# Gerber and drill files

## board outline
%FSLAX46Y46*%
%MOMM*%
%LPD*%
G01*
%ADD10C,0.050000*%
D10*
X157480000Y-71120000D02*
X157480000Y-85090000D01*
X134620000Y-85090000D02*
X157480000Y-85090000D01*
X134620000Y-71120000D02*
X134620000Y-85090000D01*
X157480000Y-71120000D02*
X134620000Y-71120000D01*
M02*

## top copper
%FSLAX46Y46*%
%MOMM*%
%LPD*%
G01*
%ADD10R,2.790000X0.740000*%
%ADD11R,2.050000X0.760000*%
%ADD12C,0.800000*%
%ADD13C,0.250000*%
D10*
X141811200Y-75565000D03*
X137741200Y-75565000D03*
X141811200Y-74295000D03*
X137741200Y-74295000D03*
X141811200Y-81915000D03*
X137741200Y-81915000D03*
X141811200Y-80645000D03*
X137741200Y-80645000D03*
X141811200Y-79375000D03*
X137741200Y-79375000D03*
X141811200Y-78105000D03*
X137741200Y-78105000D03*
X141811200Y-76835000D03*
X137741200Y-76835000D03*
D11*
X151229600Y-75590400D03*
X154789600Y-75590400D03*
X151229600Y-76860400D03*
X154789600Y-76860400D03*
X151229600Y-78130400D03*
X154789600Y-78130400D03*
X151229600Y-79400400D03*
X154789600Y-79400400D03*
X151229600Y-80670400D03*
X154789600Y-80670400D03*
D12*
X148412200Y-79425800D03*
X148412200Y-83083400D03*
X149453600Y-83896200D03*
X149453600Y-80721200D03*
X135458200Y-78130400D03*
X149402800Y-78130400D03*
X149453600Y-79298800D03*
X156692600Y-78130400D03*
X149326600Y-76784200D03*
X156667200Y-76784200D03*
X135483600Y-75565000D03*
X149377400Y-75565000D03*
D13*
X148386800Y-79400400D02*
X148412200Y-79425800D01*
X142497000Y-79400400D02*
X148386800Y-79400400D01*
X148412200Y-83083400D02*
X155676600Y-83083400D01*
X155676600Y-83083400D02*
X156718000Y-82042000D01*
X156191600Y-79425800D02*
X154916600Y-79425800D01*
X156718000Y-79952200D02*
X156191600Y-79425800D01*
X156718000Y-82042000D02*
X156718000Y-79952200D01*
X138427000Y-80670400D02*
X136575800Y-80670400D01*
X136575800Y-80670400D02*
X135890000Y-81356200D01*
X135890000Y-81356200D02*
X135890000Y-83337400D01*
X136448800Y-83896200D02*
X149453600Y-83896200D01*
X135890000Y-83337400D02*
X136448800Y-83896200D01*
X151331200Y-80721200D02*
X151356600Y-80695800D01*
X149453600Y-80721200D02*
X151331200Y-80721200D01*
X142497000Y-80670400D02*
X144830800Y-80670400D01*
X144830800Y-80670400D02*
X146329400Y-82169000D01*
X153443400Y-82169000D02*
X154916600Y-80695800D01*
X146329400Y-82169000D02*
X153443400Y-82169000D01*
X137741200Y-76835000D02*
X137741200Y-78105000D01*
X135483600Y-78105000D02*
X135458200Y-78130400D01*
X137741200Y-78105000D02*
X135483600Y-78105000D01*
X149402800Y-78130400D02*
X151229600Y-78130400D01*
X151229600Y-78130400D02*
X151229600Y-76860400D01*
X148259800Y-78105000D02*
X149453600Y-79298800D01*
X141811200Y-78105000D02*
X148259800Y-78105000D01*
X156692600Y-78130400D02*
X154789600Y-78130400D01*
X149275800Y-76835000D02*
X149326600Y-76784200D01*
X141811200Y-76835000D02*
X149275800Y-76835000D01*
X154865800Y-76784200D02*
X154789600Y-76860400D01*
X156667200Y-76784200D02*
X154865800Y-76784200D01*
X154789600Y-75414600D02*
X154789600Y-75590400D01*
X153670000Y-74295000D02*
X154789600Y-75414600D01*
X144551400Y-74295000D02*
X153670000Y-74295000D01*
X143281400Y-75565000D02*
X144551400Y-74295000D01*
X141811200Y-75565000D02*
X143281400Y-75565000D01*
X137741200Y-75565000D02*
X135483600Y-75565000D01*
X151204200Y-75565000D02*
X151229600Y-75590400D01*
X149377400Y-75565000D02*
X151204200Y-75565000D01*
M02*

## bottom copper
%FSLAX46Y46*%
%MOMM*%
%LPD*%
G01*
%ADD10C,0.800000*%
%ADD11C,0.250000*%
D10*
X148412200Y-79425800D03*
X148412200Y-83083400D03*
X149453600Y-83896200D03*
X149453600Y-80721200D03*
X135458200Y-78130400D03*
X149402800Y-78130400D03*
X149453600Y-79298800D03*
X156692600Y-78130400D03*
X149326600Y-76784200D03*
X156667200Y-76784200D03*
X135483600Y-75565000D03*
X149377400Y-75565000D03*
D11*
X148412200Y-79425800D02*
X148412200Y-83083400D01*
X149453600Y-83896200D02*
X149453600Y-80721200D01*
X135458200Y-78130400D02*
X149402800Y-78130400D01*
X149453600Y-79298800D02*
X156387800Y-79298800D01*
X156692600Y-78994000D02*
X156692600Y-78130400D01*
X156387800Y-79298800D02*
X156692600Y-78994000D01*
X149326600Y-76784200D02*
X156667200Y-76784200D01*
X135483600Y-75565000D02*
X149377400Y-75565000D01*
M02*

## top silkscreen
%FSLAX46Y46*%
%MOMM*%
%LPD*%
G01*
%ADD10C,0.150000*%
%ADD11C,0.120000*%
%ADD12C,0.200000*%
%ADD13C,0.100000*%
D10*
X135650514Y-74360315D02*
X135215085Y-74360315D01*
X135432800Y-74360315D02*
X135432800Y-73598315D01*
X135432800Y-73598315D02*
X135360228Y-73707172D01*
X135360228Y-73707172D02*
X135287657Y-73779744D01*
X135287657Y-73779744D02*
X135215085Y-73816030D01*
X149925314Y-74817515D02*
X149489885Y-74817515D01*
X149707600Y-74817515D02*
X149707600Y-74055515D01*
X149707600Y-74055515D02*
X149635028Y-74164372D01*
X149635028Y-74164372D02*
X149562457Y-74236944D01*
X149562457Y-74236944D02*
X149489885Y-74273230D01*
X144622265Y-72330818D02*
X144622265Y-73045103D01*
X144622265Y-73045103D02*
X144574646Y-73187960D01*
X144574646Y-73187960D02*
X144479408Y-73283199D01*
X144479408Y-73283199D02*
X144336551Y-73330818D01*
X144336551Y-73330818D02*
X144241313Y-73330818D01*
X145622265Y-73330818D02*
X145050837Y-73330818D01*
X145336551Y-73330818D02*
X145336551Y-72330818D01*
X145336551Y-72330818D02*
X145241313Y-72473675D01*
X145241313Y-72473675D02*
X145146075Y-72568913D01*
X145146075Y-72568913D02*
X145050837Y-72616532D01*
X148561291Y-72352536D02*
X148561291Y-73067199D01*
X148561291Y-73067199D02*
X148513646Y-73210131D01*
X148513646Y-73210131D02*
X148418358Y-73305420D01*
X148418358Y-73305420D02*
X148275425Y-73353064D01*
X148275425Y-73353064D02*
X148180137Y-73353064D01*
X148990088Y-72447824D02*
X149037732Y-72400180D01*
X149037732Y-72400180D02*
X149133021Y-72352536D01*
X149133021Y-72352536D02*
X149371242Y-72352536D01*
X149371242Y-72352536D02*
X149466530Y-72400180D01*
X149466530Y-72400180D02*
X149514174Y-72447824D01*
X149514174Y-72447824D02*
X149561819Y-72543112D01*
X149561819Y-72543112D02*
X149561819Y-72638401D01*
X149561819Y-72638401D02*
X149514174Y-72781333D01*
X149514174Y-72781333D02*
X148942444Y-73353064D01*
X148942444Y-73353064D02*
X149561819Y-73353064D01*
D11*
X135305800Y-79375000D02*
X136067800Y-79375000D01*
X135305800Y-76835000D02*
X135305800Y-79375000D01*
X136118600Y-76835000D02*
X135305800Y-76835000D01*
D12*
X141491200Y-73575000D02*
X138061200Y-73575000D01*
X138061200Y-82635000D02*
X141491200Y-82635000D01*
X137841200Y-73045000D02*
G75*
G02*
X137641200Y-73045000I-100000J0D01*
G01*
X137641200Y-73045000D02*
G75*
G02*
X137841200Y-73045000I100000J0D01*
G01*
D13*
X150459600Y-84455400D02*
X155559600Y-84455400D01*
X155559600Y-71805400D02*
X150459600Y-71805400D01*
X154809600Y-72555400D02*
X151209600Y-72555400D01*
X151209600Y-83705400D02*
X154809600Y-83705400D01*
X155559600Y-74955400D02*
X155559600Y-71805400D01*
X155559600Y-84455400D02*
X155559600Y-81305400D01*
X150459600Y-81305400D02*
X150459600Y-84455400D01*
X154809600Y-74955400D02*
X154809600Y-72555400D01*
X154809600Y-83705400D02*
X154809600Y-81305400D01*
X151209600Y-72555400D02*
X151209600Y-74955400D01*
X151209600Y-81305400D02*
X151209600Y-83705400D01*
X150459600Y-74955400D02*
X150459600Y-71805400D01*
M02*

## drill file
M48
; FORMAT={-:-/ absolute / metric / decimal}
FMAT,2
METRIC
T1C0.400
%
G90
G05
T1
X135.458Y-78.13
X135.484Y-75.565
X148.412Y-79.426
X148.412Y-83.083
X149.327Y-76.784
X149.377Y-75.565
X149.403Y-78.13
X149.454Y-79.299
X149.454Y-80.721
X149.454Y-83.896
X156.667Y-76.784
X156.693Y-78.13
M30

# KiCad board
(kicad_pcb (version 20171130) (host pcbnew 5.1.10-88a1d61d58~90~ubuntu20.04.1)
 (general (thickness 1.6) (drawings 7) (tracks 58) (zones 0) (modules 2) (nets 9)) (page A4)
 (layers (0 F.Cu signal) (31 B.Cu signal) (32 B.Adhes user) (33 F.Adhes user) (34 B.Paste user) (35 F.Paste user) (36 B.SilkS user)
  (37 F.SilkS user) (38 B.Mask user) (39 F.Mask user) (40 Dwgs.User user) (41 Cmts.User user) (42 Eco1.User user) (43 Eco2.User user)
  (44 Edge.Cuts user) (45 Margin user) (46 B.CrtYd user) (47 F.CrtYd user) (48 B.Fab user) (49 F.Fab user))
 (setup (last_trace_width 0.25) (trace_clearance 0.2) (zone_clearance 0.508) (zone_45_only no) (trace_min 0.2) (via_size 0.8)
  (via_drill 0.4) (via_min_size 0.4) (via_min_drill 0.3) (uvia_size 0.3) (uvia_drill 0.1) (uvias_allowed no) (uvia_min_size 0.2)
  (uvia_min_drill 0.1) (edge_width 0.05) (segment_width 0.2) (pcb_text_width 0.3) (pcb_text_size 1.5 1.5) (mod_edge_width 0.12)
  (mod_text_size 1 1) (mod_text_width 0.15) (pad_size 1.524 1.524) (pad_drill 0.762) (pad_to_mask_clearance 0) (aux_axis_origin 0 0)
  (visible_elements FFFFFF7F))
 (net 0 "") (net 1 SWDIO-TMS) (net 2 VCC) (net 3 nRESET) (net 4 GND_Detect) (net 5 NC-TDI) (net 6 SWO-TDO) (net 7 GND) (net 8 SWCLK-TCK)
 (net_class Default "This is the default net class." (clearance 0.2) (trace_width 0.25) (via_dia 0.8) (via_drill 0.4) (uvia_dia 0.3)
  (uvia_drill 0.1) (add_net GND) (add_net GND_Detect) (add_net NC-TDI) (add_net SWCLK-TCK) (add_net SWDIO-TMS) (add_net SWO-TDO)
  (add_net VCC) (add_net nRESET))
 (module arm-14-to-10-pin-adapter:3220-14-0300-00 (layer F.Cu) (at 139.7762 78.105 270)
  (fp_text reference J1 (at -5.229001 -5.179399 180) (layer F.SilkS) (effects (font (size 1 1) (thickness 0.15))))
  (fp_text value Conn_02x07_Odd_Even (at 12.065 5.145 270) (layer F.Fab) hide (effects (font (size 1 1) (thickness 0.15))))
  (fp_line (start 1.27 4.4704) (end 1.27 3.7084) (layer F.SilkS) (width 0.12))
  (fp_line (start -1.27 4.4704) (end 1.27 4.4704) (layer F.SilkS) (width 0.12))
  (fp_line (start -1.27 3.6576) (end -1.27 4.4704) (layer F.SilkS) (width 0.12))
  (fp_line (start -4.53 -1.715) (end -4.53 1.715) (layer F.SilkS) (width 0.2))
  (fp_line (start 4.53 1.715) (end 4.53 -1.715) (layer F.SilkS) (width 0.2))
  (fp_circle (center -5.06 2.035) (end -4.96 2.035) (layer F.SilkS) (width 0.2))
  (pad 4 smd rect (at -2.54 -2.035 270) (size 0.74 2.79) (layers F.Cu F.Paste F.Mask) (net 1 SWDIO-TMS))
  (pad 3 smd rect (at -2.54 2.035 270) (size 0.74 2.79) (layers F.Cu F.Paste F.Mask) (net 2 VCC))
  (pad 2 smd rect (at -3.81 -2.035 270) (size 0.74 2.79) (layers F.Cu F.Paste F.Mask))
  (pad 1 smd rect (at -3.81 2.035 270) (size 0.74 2.79) (layers F.Cu F.Paste F.Mask))
  (pad 14 smd rect (at 3.81 -2.035 270) (size 0.74 2.79) (layers F.Cu F.Paste F.Mask))
  (pad 13 smd rect (at 3.81 2.035 270) (size 0.74 2.79) (layers F.Cu F.Paste F.Mask))
  (pad 12 smd rect (at 2.54 -2.035 270) (size 0.74 2.79) (layers F.Cu F.Paste F.Mask) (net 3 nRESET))
  (pad 11 smd rect (at 2.54 2.035 270) (size 0.74 2.79) (layers F.Cu F.Paste F.Mask) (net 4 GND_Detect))
  (pad 10 smd rect (at 1.27 -2.035 270) (size 0.74 2.79) (layers F.Cu F.Paste F.Mask) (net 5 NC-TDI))
  (pad 9 smd rect (at 1.27 2.035 270) (size 0.74 2.79) (layers F.Cu F.Paste F.Mask))
  (pad 8 smd rect (at 0 -2.035 270) (size 0.74 2.79) (layers F.Cu F.Paste F.Mask) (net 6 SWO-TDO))
  (pad 7 smd rect (at 0 2.035 270) (size 0.74 2.79) (layers F.Cu F.Paste F.Mask) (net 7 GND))
  (pad 6 smd rect (at -1.27 -2.035 270) (size 0.74 2.79) (layers F.Cu F.Paste F.Mask) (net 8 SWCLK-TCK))
  (pad 5 smd rect (at -1.27 2.035 270) (size 0.74 2.79) (layers F.Cu F.Paste F.Mask) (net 7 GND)))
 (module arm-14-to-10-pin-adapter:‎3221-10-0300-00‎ (layer F.Cu) (at 153.0096 78.1304 270)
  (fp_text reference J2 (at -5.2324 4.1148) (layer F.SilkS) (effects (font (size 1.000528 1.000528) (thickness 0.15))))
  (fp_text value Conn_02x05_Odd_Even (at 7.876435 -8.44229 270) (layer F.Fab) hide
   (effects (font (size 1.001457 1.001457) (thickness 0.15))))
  (fp_line (start 6.325 2.55) (end 6.325 -2.55) (layer F.SilkS) (width 0.1))
  (fp_line (start -6.325 -2.55) (end -6.325 2.55) (layer F.SilkS) (width 0.1))
  (fp_line (start -5.575 -1.8) (end -5.575 1.8) (layer F.SilkS) (width 0.1))
  (fp_line (start 5.575 1.8) (end 5.575 -1.8) (layer F.SilkS) (width 0.1))
  (fp_line (start -3.175 -2.55) (end -6.325 -2.55) (layer F.SilkS) (width 0.1))
  (fp_line (start 6.325 -2.55) (end 3.175 -2.55) (layer F.SilkS) (width 0.1))
  (fp_line (start 3.175 2.55) (end 6.325 2.55) (layer F.SilkS) (width 0.1))
  (fp_line (start -3.175 -1.8) (end -5.575 -1.8) (layer F.SilkS) (width 0.1))
  (fp_line (start 5.575 -1.8) (end 3.175 -1.8) (layer F.SilkS) (width 0.1))
  (fp_line (start -5.575 1.8) (end -3.175 1.8) (layer F.SilkS) (width 0.1))
  (fp_line (start 3.175 1.8) (end 5.575 1.8) (layer F.SilkS) (width 0.1))
  (fp_line (start -3.175 2.55) (end -6.325 2.55) (layer F.SilkS) (width 0.1))
  (pad 1 smd rect (at -2.54 1.78 270) (size 0.76 2.05) (layers F.Cu F.Paste F.Mask) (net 2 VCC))
  (pad 2 smd rect (at -2.54 -1.78 270) (size 0.76 2.05) (layers F.Cu F.Paste F.Mask) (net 1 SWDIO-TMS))
  (pad 3 smd rect (at -1.27 1.78 270) (size 0.76 2.05) (layers F.Cu F.Paste F.Mask) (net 7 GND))
  (pad 4 smd rect (at -1.27 -1.78 270) (size 0.76 2.05) (layers F.Cu F.Paste F.Mask) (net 8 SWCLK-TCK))
  (pad 5 smd rect (at 0 1.78 270) (size 0.76 2.05) (layers F.Cu F.Paste F.Mask) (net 7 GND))
  (pad 6 smd rect (at 0 -1.78 270) (size 0.76 2.05) (layers F.Cu F.Paste F.Mask) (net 6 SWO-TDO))
  (pad 7 smd rect (at 1.27 1.78 270) (size 0.76 2.05) (layers F.Cu F.Paste F.Mask))
  (pad 8 smd rect (at 1.27 -1.78 270) (size 0.76 2.05) (layers F.Cu F.Paste F.Mask) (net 5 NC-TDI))
  (pad 9 smd rect (at 2.54 1.78 270) (size 0.76 2.05) (layers F.Cu F.Paste F.Mask) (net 4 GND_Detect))
  (pad 10 smd rect (at 2.54 -1.78 270) (size 0.76 2.05) (layers F.Cu F.Paste F.Mask) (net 3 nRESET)))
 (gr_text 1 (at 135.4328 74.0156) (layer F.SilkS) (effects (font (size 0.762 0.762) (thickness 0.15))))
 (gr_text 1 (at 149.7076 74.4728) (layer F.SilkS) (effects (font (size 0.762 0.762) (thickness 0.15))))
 (gr_line (start 157.48 71.12) (end 157.48 85.09) (layer Edge.Cuts) (width 0.05))
 (gr_line (start 134.62 85.09) (end 157.48 85.09) (layer Edge.Cuts) (width 0.05))
 (gr_line (start 134.62 71.12) (end 134.62 85.09) (layer Edge.Cuts) (width 0.05))
 (gr_line (start 157.48 71.12) (end 134.62 71.12) (layer Edge.Cuts) (width 0.05))
 (via (at 148.4122 79.4258) (size 0.8) (drill 0.4) (layers F.Cu B.Cu) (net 5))
 (segment (start 148.3868 79.4004) (end 148.4122 79.4258) (width 0.25) (layer F.Cu) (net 5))
 (segment (start 142.497 79.4004) (end 148.3868 79.4004) (width 0.25) (layer F.Cu) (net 5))
 (via (at 148.4122 83.0834) (size 0.8) (drill 0.4) (layers F.Cu B.Cu) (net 5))
 (segment (start 148.4122 79.4258) (end 148.4122 83.0834) (width 0.25) (layer B.Cu) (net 5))
 (segment (start 148.4122 83.0834) (end 155.6766 83.0834) (width 0.25) (layer F.Cu) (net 5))
 (segment (start 155.6766 83.0834) (end 156.718 82.042) (width 0.25) (layer F.Cu) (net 5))
 (segment (start 156.1916 79.4258) (end 154.9166 79.4258) (width 0.25) (layer F.Cu) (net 5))
 (segment (start 156.718 79.9522) (end 156.1916 79.4258) (width 0.25) (layer F.Cu) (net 5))
 (segment (start 156.718 82.042) (end 156.718 79.9522) (width 0.25) (layer F.Cu) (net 5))
 (segment (start 138.427 80.6704) (end 136.5758 80.6704) (width 0.25) (layer F.Cu) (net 4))
 (segment (start 136.5758 80.6704) (end 135.89 81.3562) (width 0.25) (layer F.Cu) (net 4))
 (segment (start 135.89 81.3562) (end 135.89 83.3374) (width 0.25) (layer F.Cu) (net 4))
 (via (at 149.4536 83.8962) (size 0.8) (drill 0.4) (layers F.Cu B.Cu) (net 4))
 (segment (start 136.4488 83.8962) (end 149.4536 83.8962) (width 0.25) (layer F.Cu) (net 4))
 (segment (start 135.89 83.3374) (end 136.4488 83.8962) (width 0.25) (layer F.Cu) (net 4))
 (via (at 149.4536 80.7212) (size 0.8) (drill 0.4) (layers F.Cu B.Cu) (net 4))
 (segment (start 149.4536 83.8962) (end 149.4536 80.7212) (width 0.25) (layer B.Cu) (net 4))
 (segment (start 151.3312 80.7212) (end 151.3566 80.6958) (width 0.25) (layer F.Cu) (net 4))
 (segment (start 149.4536 80.7212) (end 151.3312 80.7212) (width 0.25) (layer F.Cu) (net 4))
 (segment (start 142.497 80.6704) (end 144.8308 80.6704) (width 0.25) (layer F.Cu) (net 3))
 (segment (start 144.8308 80.6704) (end 146.3294 82.169) (width 0.25) (layer F.Cu) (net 3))
 (segment (start 153.4434 82.169) (end 154.9166 80.6958) (width 0.25) (layer F.Cu) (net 3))
 (segment (start 146.3294 82.169) (end 153.4434 82.169) (width 0.25) (layer F.Cu) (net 3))
 (segment (start 137.7412 76.835) (end 137.7412 78.105) (width 0.25) (layer F.Cu) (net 7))
 (segment (start 135.4836 78.105) (end 135.4582 78.1304) (width 0.25) (layer F.Cu) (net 7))
 (via (at 135.4582 78.1304) (size 0.8) (drill 0.4) (layers F.Cu B.Cu) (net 7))
 (segment (start 137.7412 78.105) (end 135.4836 78.105) (width 0.25) (layer F.Cu) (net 7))
 (via (at 149.4028 78.1304) (size 0.8) (drill 0.4) (layers F.Cu B.Cu) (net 7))
 (segment (start 135.4582 78.1304) (end 149.4028 78.1304) (width 0.25) (layer B.Cu) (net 7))
 (segment (start 149.4028 78.1304) (end 151.2296 78.1304) (width 0.25) (layer F.Cu) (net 7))
 (segment (start 151.2296 78.1304) (end 151.2296 76.8604) (width 0.25) (layer F.Cu) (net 7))
 (via (at 149.4536 79.2988) (size 0.8) (drill 0.4) (layers F.Cu B.Cu) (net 6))
 (segment (start 148.2598 78.105) (end 149.4536 79.2988) (width 0.25) (layer F.Cu) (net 6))
 (segment (start 141.8112 78.105) (end 148.2598 78.105) (width 0.25) (layer F.Cu) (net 6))
 (segment (start 149.4536 79.2988) (end 156.3878 79.2988) (width 0.25) (layer B.Cu) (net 6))
 (via (at 156.6926 78.1304) (size 0.8) (drill 0.4) (layers F.Cu B.Cu) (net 6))
 (segment (start 156.6926 78.994) (end 156.6926 78.1304) (width 0.25) (layer B.Cu) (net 6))
 (segment (start 156.3878 79.2988) (end 156.6926 78.994) (width 0.25) (layer B.Cu) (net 6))
 (segment (start 156.6926 78.1304) (end 154.7896 78.1304) (width 0.25) (layer F.Cu) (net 6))
 (via (at 149.3266 76.7842) (size 0.8) (drill 0.4) (layers F.Cu B.Cu) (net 8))
 (segment (start 149.2758 76.835) (end 149.3266 76.7842) (width 0.25) (layer F.Cu) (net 8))
 (segment (start 141.8112 76.835) (end 149.2758 76.835) (width 0.25) (layer F.Cu) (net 8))
 (via (at 156.6672 76.7842) (size 0.8) (drill 0.4) (layers F.Cu B.Cu) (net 8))
 (segment (start 149.3266 76.7842) (end 156.6672 76.7842) (width 0.25) (layer B.Cu) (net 8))
 (segment (start 154.8658 76.7842) (end 154.7896 76.8604) (width 0.25) (layer F.Cu) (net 8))
 (segment (start 156.6672 76.7842) (end 154.8658 76.7842) (width 0.25) (layer F.Cu) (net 8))
 (segment (start 154.7896 75.4146) (end 154.7896 75.5904) (width 0.25) (layer F.Cu) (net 1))
 (segment (start 153.67 74.295) (end 154.7896 75.4146) (width 0.25) (layer F.Cu) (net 1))
 (segment (start 144.5514 74.295) (end 153.67 74.295) (width 0.25) (layer F.Cu) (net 1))
 (segment (start 143.2814 75.565) (end 144.5514 74.295) (width 0.25) (layer F.Cu) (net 1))
 (segment (start 141.8112 75.565) (end 143.2814 75.565) (width 0.25) (layer F.Cu) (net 1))
 (via (at 135.4836 75.565) (size 0.8) (drill 0.4) (layers F.Cu B.Cu) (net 2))
 (segment (start 137.7412 75.565) (end 135.4836 75.565) (width 0.25) (layer F.Cu) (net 2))
 (via (at 149.3774 75.565) (size 0.8) (drill 0.4) (layers F.Cu B.Cu) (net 2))
 (segment (start 135.4836 75.565) (end 149.3774 75.565) (width 0.25) (layer B.Cu) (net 2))
 (segment (start 151.2042 75.565) (end 151.2296 75.5904) (width 0.25) (layer F.Cu) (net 2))
 (segment (start 149.3774 75.565) (end 151.2042 75.565) (width 0.25) (layer F.Cu) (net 2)))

